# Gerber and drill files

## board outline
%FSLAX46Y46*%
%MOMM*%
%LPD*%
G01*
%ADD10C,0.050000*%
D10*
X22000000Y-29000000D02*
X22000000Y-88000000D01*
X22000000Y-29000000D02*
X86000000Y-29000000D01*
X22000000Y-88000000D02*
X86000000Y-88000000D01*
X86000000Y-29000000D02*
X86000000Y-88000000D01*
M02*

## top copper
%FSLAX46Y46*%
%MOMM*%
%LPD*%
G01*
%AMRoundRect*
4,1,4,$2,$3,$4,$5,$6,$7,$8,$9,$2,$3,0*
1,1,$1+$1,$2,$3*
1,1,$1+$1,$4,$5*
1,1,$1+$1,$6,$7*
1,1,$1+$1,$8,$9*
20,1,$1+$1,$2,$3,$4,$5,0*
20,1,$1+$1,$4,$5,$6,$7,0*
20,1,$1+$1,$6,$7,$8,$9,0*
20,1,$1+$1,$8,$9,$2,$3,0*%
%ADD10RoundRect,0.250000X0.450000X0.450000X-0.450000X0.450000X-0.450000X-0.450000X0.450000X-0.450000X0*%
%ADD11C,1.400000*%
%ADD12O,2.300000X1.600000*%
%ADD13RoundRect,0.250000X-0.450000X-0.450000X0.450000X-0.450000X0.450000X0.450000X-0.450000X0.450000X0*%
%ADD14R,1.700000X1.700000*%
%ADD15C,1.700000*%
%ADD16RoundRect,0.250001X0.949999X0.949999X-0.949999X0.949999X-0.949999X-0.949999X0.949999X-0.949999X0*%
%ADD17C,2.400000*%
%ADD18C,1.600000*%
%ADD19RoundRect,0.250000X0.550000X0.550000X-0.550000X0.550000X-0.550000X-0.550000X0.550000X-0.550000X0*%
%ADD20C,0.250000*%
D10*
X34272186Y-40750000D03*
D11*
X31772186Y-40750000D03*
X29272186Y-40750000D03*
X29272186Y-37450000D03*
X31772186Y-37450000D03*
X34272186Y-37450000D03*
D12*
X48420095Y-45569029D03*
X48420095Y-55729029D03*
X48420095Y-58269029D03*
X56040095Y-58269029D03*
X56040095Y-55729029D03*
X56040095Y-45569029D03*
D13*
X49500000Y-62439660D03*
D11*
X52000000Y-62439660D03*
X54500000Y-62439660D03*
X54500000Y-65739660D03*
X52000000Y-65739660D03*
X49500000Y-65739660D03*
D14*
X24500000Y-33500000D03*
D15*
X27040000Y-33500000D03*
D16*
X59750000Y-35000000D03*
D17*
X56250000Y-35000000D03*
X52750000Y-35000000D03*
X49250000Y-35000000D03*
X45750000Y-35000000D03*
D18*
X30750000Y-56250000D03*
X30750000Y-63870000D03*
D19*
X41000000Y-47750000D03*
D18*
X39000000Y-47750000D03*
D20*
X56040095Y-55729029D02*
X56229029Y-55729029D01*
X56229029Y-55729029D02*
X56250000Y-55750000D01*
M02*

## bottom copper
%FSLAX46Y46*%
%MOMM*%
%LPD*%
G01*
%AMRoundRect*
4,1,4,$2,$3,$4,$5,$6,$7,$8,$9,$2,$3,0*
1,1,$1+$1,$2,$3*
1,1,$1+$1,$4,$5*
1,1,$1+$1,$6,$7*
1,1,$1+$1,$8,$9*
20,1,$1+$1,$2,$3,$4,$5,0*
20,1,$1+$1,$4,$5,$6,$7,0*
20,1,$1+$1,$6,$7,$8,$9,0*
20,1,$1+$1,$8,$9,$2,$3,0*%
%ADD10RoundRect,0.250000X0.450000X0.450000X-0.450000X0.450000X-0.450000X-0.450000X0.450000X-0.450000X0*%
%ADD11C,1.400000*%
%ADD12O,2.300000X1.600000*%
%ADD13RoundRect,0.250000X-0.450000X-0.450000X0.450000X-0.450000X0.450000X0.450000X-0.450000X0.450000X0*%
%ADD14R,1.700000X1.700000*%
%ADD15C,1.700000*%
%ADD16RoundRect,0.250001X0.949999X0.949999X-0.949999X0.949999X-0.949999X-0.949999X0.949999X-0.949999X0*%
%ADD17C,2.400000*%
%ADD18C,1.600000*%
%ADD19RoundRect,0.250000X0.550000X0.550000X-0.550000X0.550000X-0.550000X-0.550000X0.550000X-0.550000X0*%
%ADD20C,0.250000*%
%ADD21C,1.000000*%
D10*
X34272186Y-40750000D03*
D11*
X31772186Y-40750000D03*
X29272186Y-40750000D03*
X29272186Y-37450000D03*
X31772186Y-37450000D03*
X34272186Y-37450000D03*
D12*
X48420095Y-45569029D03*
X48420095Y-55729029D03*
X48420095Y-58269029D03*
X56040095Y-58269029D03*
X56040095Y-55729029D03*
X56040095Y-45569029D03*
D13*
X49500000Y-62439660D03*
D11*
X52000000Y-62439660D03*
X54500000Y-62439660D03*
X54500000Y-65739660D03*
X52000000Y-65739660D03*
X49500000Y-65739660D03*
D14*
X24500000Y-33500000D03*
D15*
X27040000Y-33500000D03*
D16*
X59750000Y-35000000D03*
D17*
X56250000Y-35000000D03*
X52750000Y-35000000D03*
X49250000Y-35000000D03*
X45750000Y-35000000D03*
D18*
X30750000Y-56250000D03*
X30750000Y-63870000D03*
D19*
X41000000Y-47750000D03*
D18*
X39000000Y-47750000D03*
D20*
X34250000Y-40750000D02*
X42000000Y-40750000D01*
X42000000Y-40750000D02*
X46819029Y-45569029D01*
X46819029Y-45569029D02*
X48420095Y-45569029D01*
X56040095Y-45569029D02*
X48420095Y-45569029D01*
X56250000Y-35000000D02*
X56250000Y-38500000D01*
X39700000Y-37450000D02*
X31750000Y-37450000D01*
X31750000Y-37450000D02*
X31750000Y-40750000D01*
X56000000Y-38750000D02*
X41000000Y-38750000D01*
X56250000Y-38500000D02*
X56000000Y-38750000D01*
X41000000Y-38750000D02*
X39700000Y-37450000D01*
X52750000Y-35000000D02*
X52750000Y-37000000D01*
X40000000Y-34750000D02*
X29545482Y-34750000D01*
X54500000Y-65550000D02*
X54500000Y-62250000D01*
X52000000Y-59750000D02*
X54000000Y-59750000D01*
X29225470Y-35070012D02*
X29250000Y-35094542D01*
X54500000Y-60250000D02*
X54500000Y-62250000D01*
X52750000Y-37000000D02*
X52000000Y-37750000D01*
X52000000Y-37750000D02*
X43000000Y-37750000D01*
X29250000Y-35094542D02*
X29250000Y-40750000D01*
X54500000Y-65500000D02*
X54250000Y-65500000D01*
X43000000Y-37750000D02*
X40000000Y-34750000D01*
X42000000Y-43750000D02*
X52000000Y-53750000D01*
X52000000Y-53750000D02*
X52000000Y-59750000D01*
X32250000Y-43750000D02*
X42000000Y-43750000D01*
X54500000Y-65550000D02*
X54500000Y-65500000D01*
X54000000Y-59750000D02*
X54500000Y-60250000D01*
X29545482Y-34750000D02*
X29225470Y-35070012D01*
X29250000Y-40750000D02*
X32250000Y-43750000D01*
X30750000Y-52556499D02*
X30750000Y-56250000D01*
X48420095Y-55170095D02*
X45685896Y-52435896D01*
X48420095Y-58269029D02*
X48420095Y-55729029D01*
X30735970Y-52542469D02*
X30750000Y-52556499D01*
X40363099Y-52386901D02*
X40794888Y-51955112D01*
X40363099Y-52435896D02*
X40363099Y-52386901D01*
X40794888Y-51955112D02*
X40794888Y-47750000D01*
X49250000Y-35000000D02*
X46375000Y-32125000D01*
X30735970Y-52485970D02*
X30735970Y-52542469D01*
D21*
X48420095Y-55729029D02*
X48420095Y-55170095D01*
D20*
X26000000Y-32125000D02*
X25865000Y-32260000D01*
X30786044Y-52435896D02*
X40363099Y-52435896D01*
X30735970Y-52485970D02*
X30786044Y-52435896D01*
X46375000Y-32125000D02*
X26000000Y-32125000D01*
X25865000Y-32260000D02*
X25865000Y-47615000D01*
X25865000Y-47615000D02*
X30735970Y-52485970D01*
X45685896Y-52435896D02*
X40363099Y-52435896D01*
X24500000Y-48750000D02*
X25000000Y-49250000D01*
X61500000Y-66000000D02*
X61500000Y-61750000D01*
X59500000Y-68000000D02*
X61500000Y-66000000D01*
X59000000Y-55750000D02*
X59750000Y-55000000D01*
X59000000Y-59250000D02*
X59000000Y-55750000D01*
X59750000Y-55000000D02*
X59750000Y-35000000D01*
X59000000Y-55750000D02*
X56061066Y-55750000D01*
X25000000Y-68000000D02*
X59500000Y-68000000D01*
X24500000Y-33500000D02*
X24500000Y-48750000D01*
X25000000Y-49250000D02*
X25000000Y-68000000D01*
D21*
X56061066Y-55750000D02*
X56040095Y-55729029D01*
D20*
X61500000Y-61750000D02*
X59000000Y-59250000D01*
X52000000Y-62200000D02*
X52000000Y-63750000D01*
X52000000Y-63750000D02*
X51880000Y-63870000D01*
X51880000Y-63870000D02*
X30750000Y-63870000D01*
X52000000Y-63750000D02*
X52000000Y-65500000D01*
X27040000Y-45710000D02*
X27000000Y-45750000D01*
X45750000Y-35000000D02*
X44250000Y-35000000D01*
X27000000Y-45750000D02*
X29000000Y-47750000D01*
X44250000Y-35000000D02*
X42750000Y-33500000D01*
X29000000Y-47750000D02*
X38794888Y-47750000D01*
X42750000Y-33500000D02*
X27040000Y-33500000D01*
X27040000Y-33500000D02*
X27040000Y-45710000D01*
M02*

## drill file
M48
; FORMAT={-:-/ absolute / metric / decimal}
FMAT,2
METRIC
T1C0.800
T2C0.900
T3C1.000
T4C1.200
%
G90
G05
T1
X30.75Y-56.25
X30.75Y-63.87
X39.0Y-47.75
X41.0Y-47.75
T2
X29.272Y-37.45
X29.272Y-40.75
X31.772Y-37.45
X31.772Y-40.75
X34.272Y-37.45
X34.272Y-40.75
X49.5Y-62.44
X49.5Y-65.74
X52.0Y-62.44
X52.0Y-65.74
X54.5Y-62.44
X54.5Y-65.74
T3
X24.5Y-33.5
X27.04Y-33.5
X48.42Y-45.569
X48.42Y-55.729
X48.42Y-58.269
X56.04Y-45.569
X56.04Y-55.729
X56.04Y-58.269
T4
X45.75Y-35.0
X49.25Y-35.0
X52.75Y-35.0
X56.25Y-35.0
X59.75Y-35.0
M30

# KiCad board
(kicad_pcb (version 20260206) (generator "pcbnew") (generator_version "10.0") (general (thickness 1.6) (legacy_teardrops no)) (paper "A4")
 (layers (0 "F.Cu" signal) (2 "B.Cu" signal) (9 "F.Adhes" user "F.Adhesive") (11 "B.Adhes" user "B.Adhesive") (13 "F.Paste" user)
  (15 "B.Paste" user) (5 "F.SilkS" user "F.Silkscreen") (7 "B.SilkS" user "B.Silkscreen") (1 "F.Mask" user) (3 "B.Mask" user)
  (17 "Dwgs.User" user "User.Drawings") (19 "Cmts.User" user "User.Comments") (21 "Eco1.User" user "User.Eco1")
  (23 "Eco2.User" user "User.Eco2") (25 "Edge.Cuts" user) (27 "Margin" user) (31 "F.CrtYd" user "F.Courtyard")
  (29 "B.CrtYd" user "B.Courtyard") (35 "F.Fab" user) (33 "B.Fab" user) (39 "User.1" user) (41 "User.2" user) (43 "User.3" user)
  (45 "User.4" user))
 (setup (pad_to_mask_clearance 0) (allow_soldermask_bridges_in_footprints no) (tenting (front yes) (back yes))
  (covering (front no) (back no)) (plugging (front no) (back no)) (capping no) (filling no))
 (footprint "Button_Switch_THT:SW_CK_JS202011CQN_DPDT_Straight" (layer "F.Cu") (at 34.272186 40.75 180)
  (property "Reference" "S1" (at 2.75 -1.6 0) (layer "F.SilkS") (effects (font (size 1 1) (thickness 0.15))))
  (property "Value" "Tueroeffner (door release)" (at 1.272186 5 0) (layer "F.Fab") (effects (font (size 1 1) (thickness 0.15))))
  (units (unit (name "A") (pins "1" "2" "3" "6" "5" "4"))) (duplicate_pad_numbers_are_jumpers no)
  (pad "1" thru_hole roundrect (at 0 0 180) (size 1.4 1.4) (drill 0.9) (layers "*.Cu" "*.Mask") (remove_unused_layers no)
   (roundrect_rratio 0.1785714286) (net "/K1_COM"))
  (pad "2" thru_hole circle (at 2.5 0 180) (size 1.4 1.4) (drill 0.9) (layers "*.Cu" "*.Mask") (remove_unused_layers no) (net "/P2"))
  (pad "3" thru_hole circle (at 5 0 180) (size 1.4 1.4) (drill 0.9) (layers "*.Cu" "*.Mask") (remove_unused_layers no) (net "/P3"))
  (pad "4" thru_hole circle (at 5 3.3 180) (size 1.4 1.4) (drill 0.9) (layers "*.Cu" "*.Mask") (remove_unused_layers no) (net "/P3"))
  (pad "5" thru_hole circle (at 2.5 3.3 180) (size 1.4 1.4) (drill 0.9) (layers "*.Cu" "*.Mask") (remove_unused_layers no) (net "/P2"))
  (pad "6" thru_hole circle (at 0 3.3 180) (size 1.4 1.4) (drill 0.9) (layers "*.Cu" "*.Mask") (remove_unused_layers no) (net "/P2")))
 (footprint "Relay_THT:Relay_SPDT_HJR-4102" (layer "F.Cu") (at 48.420095 45.569029)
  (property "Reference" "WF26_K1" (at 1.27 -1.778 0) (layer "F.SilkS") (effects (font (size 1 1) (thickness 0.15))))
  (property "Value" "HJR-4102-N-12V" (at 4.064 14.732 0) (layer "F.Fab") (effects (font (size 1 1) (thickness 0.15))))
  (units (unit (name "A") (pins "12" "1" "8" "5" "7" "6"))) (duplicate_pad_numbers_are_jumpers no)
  (pad "1" thru_hole oval (at 0 0) (size 2.3 1.6) (drill 1) (layers "*.Cu" "*.Mask") (remove_unused_layers no) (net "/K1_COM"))
  (pad "5" thru_hole oval (at 0 10.16) (size 2.3 1.6) (drill 1) (layers "*.Cu" "*.Mask") (remove_unused_layers no) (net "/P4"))
  (pad "6" thru_hole oval (at 0 12.7) (size 2.3 1.6) (drill 1) (layers "*.Cu" "*.Mask") (remove_unused_layers no) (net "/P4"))
  (pad "7" thru_hole oval (at 7.62 12.7) (size 2.3 1.6) (drill 1) (layers "*.Cu" "*.Mask") (remove_unused_layers no)
   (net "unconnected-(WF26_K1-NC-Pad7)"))
  (pad "8" thru_hole oval (at 7.62 10.16) (size 2.3 1.6) (drill 1) (layers "*.Cu" "*.Mask") (remove_unused_layers no) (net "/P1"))
  (pad "12" thru_hole oval (at 7.62 0) (size 2.3 1.6) (drill 1) (layers "*.Cu" "*.Mask") (remove_unused_layers no) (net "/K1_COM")))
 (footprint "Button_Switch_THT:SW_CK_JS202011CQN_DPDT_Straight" (layer "F.Cu") (at 49.5 62.43966)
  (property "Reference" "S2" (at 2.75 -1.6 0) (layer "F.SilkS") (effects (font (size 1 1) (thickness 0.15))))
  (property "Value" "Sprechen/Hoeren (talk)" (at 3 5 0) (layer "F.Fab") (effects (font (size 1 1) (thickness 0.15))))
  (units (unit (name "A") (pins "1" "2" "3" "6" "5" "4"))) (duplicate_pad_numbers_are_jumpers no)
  (pad "1" thru_hole roundrect (at 0 0) (size 1.4 1.4) (drill 0.9) (layers "*.Cu" "*.Mask") (remove_unused_layers no)
   (roundrect_rratio 0.1785714286) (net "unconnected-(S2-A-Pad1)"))
  (pad "2" thru_hole circle (at 2.5 0) (size 1.4 1.4) (drill 0.9) (layers "*.Cu" "*.Mask") (remove_unused_layers no) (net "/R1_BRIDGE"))
  (pad "3" thru_hole circle (at 5 0) (size 1.4 1.4) (drill 0.9) (layers "*.Cu" "*.Mask") (remove_unused_layers no) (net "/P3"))
  (pad "4" thru_hole circle (at 5 3.3) (size 1.4 1.4) (drill 0.9) (layers "*.Cu" "*.Mask") (remove_unused_layers no) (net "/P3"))
  (pad "5" thru_hole circle (at 2.5 3.3) (size 1.4 1.4) (drill 0.9) (layers "*.Cu" "*.Mask") (remove_unused_layers no) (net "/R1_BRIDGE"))
  (pad "6" thru_hole circle (at 0 3.3) (size 1.4 1.4) (drill 0.9) (layers "*.Cu" "*.Mask") (remove_unused_layers no)
   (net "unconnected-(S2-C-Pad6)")))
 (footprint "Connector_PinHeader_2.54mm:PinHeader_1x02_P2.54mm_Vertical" (layer "F.Cu") (at 24.5 33.5 90)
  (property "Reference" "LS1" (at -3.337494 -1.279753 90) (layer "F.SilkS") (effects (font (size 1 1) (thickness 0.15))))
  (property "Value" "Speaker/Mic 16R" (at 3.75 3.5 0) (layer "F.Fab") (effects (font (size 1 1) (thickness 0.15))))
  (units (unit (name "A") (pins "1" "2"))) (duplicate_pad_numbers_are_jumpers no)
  (pad "1" thru_hole rect (at 0 0 90) (size 1.7 1.7) (drill 1) (layers "*.Cu" "*.Mask") (remove_unused_layers no) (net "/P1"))
  (pad "2" thru_hole circle (at 0 2.54 90) (size 1.7 1.7) (drill 1) (layers "*.Cu" "*.Mask") (remove_unused_layers no) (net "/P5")))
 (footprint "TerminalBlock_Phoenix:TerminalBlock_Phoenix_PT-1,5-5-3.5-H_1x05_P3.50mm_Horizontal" (layer "F.Cu") (at 59.75 35 180)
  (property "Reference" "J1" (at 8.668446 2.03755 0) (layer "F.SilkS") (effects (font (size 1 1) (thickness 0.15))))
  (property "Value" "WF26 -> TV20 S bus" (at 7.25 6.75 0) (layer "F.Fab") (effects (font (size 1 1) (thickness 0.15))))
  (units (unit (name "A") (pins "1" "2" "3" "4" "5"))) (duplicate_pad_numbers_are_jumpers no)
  (pad "1" thru_hole roundrect (at 0 0 180) (size 2.4 2.4) (drill 1.2) (layers "*.Cu" "*.Mask") (remove_unused_layers no)
   (roundrect_rratio 0.104167) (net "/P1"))
  (pad "2" thru_hole circle (at 3.5 0 180) (size 2.4 2.4) (drill 1.2) (layers "*.Cu" "*.Mask") (remove_unused_layers no) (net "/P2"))
  (pad "3" thru_hole circle (at 7 0 180) (size 2.4 2.4) (drill 1.2) (layers "*.Cu" "*.Mask") (remove_unused_layers no) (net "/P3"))
  (pad "4" thru_hole circle (at 10.5 0 180) (size 2.4 2.4) (drill 1.2) (layers "*.Cu" "*.Mask") (remove_unused_layers no) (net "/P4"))
  (pad "5" thru_hole circle (at 14 0 180) (size 2.4 2.4) (drill 1.2) (layers "*.Cu" "*.Mask") (remove_unused_layers no) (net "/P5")))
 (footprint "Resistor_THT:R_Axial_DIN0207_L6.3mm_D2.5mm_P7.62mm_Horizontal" (layer "F.Cu") (at 30.75 56.25 -90)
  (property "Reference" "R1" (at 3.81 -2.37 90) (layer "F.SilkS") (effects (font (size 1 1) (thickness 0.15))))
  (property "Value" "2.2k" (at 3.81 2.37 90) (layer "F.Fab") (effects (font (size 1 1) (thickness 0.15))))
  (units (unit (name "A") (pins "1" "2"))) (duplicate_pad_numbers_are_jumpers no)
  (pad "1" thru_hole circle (at 0 0 270) (size 1.6 1.6) (drill 0.8) (layers "*.Cu" "*.Mask") (remove_unused_layers no) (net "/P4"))
  (pad "2" thru_hole circle (at 7.62 0 270) (size 1.6 1.6) (drill 0.8) (layers "*.Cu" "*.Mask") (remove_unused_layers no) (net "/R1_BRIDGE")))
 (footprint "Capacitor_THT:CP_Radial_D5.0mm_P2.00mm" (layer "F.Cu") (at 41 47.75 180)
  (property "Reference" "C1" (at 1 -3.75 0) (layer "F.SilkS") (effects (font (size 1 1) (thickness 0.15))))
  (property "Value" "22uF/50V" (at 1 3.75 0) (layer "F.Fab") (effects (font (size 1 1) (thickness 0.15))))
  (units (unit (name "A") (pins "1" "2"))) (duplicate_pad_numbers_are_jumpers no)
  (pad "1" thru_hole roundrect (at 0 0 180) (size 1.6 1.6) (drill 0.8) (layers "*.Cu" "*.Mask") (remove_unused_layers no)
   (roundrect_rratio 0.15625) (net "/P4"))
  (pad "2" thru_hole circle (at 2 0 180) (size 1.6 1.6) (drill 0.8) (layers "*.Cu" "*.Mask") (remove_unused_layers no) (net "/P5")))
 (gr_line (start 22 29) (end 22 88) (stroke (width 0.05) (type default)) (layer "Edge.Cuts"))
 (gr_line (start 22 29) (end 86 29) (stroke (width 0.05) (type default)) (layer "Edge.Cuts"))
 (gr_line (start 22 88) (end 86 88) (stroke (width 0.05) (type default)) (layer "Edge.Cuts"))
 (gr_line (start 86 29) (end 86 88) (stroke (width 0.05) (type default)) (layer "Edge.Cuts"))
 (segment (start 34.25 40.75) (end 42 40.75) (width 0.25) (layer "B.Cu") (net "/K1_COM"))
 (segment (start 42 40.75) (end 46.819029 45.569029) (width 0.25) (layer "B.Cu") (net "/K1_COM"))
 (segment (start 46.819029 45.569029) (end 48.420095 45.569029) (width 0.25) (layer "B.Cu") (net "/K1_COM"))
 (segment (start 56.040095 45.569029) (end 48.420095 45.569029) (width 0.25) (layer "B.Cu") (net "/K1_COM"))
 (segment (start 56.25 35) (end 56.25 38.5) (width 0.25) (layer "B.Cu") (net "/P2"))
 (segment (start 39.7 37.45) (end 31.75 37.45) (width 0.25) (layer "B.Cu") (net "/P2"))
 (segment (start 31.75 37.45) (end 31.75 40.75) (width 0.25) (layer "B.Cu") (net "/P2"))
 (segment (start 56 38.75) (end 41 38.75) (width 0.25) (layer "B.Cu") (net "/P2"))
 (segment (start 56.25 38.5) (end 56 38.75) (width 0.25) (layer "B.Cu") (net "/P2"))
 (segment (start 41 38.75) (end 39.7 37.45) (width 0.25) (layer "B.Cu") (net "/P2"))
 (segment (start 52.75 35) (end 52.75 37) (width 0.25) (layer "B.Cu") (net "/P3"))
 (segment (start 40 34.75) (end 29.545482 34.75) (width 0.25) (layer "B.Cu") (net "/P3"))
 (segment (start 54.5 65.55) (end 54.5 62.25) (width 0.25) (layer "B.Cu") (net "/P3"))
 (segment (start 52 59.75) (end 54 59.75) (width 0.25) (layer "B.Cu") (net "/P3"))
 (segment (start 29.22547 35.070012) (end 29.25 35.094542) (width 0.25) (layer "B.Cu") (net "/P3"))
 (segment (start 54.5 60.25) (end 54.5 62.25) (width 0.25) (layer "B.Cu") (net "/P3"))
 (segment (start 52.75 37) (end 52 37.75) (width 0.25) (layer "B.Cu") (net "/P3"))
 (segment (start 52 37.75) (end 43 37.75) (width 0.25) (layer "B.Cu") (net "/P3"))
 (segment (start 29.25 35.094542) (end 29.25 40.75) (width 0.25) (layer "B.Cu") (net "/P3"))
 (segment (start 54.5 65.5) (end 54.25 65.5) (width 0.25) (layer "B.Cu") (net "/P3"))
 (segment (start 43 37.75) (end 40 34.75) (width 0.25) (layer "B.Cu") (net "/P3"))
 (segment (start 42 43.75) (end 52 53.75) (width 0.25) (layer "B.Cu") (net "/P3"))
 (segment (start 52 53.75) (end 52 59.75) (width 0.25) (layer "B.Cu") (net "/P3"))
 (segment (start 32.25 43.75) (end 42 43.75) (width 0.25) (layer "B.Cu") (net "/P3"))
 (segment (start 54.5 65.55) (end 54.5 65.5) (width 0.25) (layer "B.Cu") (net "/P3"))
 (segment (start 54 59.75) (end 54.5 60.25) (width 0.25) (layer "B.Cu") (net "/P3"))
 (segment (start 29.545482 34.75) (end 29.22547 35.070012) (width 0.25) (layer "B.Cu") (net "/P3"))
 (segment (start 29.25 40.75) (end 32.25 43.75) (width 0.25) (layer "B.Cu") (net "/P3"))
 (segment (start 30.75 52.556499) (end 30.75 56.25) (width 0.25) (layer "B.Cu") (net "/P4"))
 (segment (start 48.420095 55.170095) (end 45.685896 52.435896) (width 0.25) (layer "B.Cu") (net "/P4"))
 (segment (start 48.420095 58.269029) (end 48.420095 55.729029) (width 0.25) (layer "B.Cu") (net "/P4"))
 (segment (start 30.73597 52.542469) (end 30.75 52.556499) (width 0.25) (layer "B.Cu") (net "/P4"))
 (segment (start 40.363099 52.386901) (end 40.794888 51.955112) (width 0.25) (layer "B.Cu") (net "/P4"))
 (segment (start 40.363099 52.435896) (end 40.363099 52.386901) (width 0.25) (layer "B.Cu") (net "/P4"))
 (segment (start 40.794888 51.955112) (end 40.794888 47.75) (width 0.25) (layer "B.Cu") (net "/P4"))
 (segment (start 49.25 35) (end 46.375 32.125) (width 0.25) (layer "B.Cu") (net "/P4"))
 (segment (start 30.73597 52.48597) (end 30.73597 52.542469) (width 0.25) (layer "B.Cu") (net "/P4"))
 (segment (start 48.420095 55.729029) (end 48.420095 55.170095) (width 1) (layer "B.Cu") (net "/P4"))
 (segment (start 26 32.125) (end 25.865 32.26) (width 0.25) (layer "B.Cu") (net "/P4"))
 (segment (start 30.786044 52.435896) (end 40.363099 52.435896) (width 0.25) (layer "B.Cu") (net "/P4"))
 (segment (start 30.73597 52.48597) (end 30.786044 52.435896) (width 0.25) (layer "B.Cu") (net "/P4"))
 (segment (start 46.375 32.125) (end 26 32.125) (width 0.25) (layer "B.Cu") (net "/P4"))
 (segment (start 25.865 32.26) (end 25.865 47.615) (width 0.25) (layer "B.Cu") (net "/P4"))
 (segment (start 25.865 47.615) (end 30.73597 52.48597) (width 0.25) (layer "B.Cu") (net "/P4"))
 (segment (start 45.685896 52.435896) (end 40.363099 52.435896) (width 0.25) (layer "B.Cu") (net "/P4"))
 (segment (start 56.040095 55.729029) (end 56.229029 55.729029) (width 0.25) (layer "F.Cu") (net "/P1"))
 (segment (start 56.229029 55.729029) (end 56.25 55.75) (width 0.25) (layer "F.Cu") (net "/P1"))
 (segment (start 24.5 48.75) (end 25 49.25) (width 0.25) (layer "B.Cu") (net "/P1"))
 (segment (start 61.5 66) (end 61.5 61.75) (width 0.25) (layer "B.Cu") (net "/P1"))
 (segment (start 59.5 68) (end 61.5 66) (width 0.25) (layer "B.Cu") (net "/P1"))
 (segment (start 59 55.75) (end 59.75 55) (width 0.25) (layer "B.Cu") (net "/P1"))
 (segment (start 59 59.25) (end 59 55.75) (width 0.25) (layer "B.Cu") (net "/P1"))
 (segment (start 59.75 55) (end 59.75 35) (width 0.25) (layer "B.Cu") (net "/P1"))
 (segment (start 59 55.75) (end 56.061066 55.75) (width 0.25) (layer "B.Cu") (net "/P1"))
 (segment (start 25 68) (end 59.5 68) (width 0.25) (layer "B.Cu") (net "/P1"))
 (segment (start 24.5 33.5) (end 24.5 48.75) (width 0.25) (layer "B.Cu") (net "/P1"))
 (segment (start 25 49.25) (end 25 68) (width 0.25) (layer "B.Cu") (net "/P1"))
 (segment (start 56.061066 55.75) (end 56.040095 55.729029) (width 1) (layer "B.Cu") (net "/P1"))
 (segment (start 61.5 61.75) (end 59 59.25) (width 0.25) (layer "B.Cu") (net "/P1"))
 (segment (start 52 62.2) (end 52 63.75) (width 0.25) (layer "B.Cu") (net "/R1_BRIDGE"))
 (segment (start 52 63.75) (end 51.88 63.87) (width 0.25) (layer "B.Cu") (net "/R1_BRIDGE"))
 (segment (start 51.88 63.87) (end 30.75 63.87) (width 0.25) (layer "B.Cu") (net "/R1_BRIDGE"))
 (segment (start 52 63.75) (end 52 65.5) (width 0.25) (layer "B.Cu") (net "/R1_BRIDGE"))
 (segment (start 27.04 45.71) (end 27 45.75) (width 0.25) (layer "B.Cu") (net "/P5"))
 (segment (start 45.75 35) (end 44.25 35) (width 0.25) (layer "B.Cu") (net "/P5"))
 (segment (start 27 45.75) (end 29 47.75) (width 0.25) (layer "B.Cu") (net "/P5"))
 (segment (start 44.25 35) (end 42.75 33.5) (width 0.25) (layer "B.Cu") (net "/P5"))
 (segment (start 29 47.75) (end 38.794888 47.75) (width 0.25) (layer "B.Cu") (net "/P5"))
 (segment (start 42.75 33.5) (end 27.04 33.5) (width 0.25) (layer "B.Cu") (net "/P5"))
 (segment (start 27.04 33.5) (end 27.04 45.71) (width 0.25) (layer "B.Cu") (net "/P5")))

